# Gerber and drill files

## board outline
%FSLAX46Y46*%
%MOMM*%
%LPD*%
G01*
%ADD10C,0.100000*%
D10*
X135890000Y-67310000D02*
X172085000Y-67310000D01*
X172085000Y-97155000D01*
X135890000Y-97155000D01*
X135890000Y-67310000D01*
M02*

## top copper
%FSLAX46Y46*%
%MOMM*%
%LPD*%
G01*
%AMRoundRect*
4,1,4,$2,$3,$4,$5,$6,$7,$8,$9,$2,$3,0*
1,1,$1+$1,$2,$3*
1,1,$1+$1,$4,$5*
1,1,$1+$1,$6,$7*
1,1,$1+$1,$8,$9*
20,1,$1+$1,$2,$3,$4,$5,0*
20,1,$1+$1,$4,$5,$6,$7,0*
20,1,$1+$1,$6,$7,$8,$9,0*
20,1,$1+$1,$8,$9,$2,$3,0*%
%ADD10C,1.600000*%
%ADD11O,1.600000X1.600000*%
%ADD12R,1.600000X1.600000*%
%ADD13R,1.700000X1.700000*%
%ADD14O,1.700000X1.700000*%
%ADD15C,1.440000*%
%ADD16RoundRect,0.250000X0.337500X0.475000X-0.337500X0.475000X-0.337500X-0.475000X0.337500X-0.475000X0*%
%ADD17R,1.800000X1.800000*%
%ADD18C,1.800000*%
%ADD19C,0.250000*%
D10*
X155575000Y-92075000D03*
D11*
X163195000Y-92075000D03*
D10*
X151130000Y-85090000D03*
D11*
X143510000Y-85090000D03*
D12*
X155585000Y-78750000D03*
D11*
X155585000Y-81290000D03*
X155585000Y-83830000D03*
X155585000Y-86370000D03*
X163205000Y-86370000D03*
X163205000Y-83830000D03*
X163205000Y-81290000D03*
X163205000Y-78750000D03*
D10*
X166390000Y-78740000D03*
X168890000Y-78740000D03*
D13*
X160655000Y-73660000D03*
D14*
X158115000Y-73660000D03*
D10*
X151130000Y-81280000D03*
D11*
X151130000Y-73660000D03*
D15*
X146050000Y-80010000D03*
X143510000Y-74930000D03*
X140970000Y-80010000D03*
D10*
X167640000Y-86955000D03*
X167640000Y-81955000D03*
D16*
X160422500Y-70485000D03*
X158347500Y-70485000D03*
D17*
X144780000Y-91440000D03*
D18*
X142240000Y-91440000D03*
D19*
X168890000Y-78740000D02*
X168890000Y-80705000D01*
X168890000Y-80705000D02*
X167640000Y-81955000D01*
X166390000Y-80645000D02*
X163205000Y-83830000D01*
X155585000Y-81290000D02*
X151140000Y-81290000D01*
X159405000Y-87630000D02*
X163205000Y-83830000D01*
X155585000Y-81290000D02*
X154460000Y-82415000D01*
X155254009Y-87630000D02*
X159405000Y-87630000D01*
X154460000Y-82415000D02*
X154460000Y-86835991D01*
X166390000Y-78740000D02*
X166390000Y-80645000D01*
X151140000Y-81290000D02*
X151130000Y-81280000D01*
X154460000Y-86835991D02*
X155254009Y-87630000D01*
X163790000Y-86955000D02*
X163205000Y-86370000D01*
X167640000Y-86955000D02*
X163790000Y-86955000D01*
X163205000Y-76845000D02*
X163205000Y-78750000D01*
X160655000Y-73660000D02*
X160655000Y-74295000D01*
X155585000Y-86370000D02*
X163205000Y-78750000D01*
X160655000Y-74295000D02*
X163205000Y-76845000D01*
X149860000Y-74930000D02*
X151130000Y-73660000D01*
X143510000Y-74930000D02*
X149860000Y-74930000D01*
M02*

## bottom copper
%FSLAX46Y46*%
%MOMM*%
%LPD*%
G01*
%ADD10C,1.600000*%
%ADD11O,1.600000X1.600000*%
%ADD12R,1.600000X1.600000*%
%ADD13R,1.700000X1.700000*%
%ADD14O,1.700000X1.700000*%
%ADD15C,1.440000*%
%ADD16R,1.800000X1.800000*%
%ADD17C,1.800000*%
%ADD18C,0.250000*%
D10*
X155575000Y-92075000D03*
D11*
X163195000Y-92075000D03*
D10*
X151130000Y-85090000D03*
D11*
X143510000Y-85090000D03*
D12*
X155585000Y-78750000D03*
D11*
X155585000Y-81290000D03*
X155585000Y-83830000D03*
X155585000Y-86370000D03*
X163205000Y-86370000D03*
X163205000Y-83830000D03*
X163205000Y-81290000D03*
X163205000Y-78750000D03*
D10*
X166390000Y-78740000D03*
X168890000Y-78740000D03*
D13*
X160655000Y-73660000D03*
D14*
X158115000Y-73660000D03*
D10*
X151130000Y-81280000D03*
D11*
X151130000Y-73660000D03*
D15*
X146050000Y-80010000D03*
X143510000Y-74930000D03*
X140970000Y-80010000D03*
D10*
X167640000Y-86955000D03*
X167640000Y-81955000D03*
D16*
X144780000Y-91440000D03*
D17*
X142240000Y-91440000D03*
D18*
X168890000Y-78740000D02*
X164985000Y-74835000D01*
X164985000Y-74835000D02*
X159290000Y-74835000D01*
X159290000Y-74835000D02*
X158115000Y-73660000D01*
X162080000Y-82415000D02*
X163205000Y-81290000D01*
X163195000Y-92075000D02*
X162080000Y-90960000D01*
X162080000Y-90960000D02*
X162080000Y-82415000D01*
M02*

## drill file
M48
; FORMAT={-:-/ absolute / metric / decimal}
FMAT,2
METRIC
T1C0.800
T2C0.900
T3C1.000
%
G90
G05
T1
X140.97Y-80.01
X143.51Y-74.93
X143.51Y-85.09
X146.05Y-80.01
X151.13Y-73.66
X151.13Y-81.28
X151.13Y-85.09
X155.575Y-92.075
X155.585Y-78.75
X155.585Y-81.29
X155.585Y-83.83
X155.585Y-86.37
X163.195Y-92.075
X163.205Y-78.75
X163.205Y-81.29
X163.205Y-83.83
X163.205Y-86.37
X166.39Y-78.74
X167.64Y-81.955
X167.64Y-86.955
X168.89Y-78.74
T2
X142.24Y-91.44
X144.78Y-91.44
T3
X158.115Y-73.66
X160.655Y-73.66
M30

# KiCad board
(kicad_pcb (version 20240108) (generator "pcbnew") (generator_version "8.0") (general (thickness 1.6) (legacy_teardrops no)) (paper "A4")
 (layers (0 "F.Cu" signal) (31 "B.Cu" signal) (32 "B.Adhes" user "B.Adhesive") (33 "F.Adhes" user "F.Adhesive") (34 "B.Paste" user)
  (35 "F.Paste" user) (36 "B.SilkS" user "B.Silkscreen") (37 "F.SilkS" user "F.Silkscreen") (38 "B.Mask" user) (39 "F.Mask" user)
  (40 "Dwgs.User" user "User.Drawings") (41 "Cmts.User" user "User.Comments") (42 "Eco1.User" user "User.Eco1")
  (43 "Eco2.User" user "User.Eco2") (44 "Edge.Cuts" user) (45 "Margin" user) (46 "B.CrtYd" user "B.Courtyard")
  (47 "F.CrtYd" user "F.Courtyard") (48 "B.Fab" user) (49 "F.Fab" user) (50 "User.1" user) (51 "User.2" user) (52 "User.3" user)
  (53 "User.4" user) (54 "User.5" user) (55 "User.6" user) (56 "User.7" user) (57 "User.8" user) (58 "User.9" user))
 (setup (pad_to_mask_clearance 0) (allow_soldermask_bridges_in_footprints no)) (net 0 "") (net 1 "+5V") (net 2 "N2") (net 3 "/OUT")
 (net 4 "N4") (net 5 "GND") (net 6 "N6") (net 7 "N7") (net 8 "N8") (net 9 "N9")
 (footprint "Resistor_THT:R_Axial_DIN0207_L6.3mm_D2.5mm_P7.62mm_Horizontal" (layer "F.Cu") (at 155.575 92.075)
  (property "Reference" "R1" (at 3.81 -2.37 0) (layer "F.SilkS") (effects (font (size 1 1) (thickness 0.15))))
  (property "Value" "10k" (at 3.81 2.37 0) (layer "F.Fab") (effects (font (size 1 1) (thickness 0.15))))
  (pad "1" thru_hole circle (at 0 0) (size 1.6 1.6) (drill 0.8) (layers "*.Cu" "*.Mask") (remove_unused_layers no) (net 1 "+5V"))
  (pad "2" thru_hole oval (at 7.62 0) (size 1.6 1.6) (drill 0.8) (layers "*.Cu" "*.Mask") (remove_unused_layers no) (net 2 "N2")))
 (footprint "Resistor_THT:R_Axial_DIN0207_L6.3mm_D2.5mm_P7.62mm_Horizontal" (layer "F.Cu") (at 151.13 85.09 180)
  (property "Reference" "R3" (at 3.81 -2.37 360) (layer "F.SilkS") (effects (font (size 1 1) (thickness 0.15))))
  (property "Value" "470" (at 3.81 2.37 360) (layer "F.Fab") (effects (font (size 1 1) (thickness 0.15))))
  (pad "1" thru_hole circle (at 0 0 180) (size 1.6 1.6) (drill 0.8) (layers "*.Cu" "*.Mask") (remove_unused_layers no) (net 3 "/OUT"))
  (pad "2" thru_hole oval (at 7.62 0 180) (size 1.6 1.6) (drill 0.8) (layers "*.Cu" "*.Mask") (remove_unused_layers no) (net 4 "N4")))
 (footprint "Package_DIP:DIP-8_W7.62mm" (layer "F.Cu") (at 155.585 78.75)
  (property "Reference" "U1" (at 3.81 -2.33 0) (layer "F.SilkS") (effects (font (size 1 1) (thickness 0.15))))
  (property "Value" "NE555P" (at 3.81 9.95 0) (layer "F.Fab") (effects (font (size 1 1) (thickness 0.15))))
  (pad "1" thru_hole rect (at 0 0) (size 1.6 1.6) (drill 0.8) (layers "*.Cu" "*.Mask") (remove_unused_layers no) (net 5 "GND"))
  (pad "2" thru_hole oval (at 0 2.54) (size 1.6 1.6) (drill 0.8) (layers "*.Cu" "*.Mask") (remove_unused_layers no) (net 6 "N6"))
  (pad "3" thru_hole oval (at 0 5.08) (size 1.6 1.6) (drill 0.8) (layers "*.Cu" "*.Mask") (remove_unused_layers no) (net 3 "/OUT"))
  (pad "4" thru_hole oval (at 0 7.62) (size 1.6 1.6) (drill 0.8) (layers "*.Cu" "*.Mask") (remove_unused_layers no) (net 1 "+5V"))
  (pad "5" thru_hole oval (at 7.62 7.62) (size 1.6 1.6) (drill 0.8) (layers "*.Cu" "*.Mask") (remove_unused_layers no) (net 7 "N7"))
  (pad "6" thru_hole oval (at 7.62 5.08) (size 1.6 1.6) (drill 0.8) (layers "*.Cu" "*.Mask") (remove_unused_layers no) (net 6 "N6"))
  (pad "7" thru_hole oval (at 7.62 2.54) (size 1.6 1.6) (drill 0.8) (layers "*.Cu" "*.Mask") (remove_unused_layers no) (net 2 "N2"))
  (pad "8" thru_hole oval (at 7.62 0) (size 1.6 1.6) (drill 0.8) (layers "*.Cu" "*.Mask") (remove_unused_layers no) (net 1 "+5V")))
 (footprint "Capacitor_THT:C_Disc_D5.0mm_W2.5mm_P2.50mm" (layer "F.Cu") (at 166.39 78.74)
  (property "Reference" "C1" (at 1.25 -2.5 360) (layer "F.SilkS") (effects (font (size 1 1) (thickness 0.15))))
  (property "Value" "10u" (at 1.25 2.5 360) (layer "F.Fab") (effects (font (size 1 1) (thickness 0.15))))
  (pad "1" thru_hole circle (at 0 0) (size 1.6 1.6) (drill 0.8) (layers "*.Cu" "*.Mask") (remove_unused_layers no) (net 6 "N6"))
  (pad "2" thru_hole circle (at 2.5 0) (size 1.6 1.6) (drill 0.8) (layers "*.Cu" "*.Mask") (remove_unused_layers no) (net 5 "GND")))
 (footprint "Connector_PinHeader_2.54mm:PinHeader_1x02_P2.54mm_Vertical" (layer "F.Cu") (at 160.655 73.66 -90)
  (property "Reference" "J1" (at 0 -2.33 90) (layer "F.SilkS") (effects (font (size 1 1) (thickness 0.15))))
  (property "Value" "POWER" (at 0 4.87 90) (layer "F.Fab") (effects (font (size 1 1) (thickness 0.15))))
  (pad "1" thru_hole rect (at 0 0 270) (size 1.7 1.7) (drill 1) (layers "*.Cu" "*.Mask") (remove_unused_layers no) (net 1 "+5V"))
  (pad "2" thru_hole oval (at 0 2.54 270) (size 1.7 1.7) (drill 1) (layers "*.Cu" "*.Mask") (remove_unused_layers no) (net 5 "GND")))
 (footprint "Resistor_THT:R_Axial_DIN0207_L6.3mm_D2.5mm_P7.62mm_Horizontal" (layer "F.Cu") (at 151.13 81.28 90)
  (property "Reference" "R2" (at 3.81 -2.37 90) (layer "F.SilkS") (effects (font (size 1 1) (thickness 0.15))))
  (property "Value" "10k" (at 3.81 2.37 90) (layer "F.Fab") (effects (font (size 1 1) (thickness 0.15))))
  (pad "1" thru_hole circle (at 0 0 90) (size 1.6 1.6) (drill 0.8) (layers "*.Cu" "*.Mask") (remove_unused_layers no) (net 6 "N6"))
  (pad "2" thru_hole oval (at 7.62 0 90) (size 1.6 1.6) (drill 0.8) (layers "*.Cu" "*.Mask") (remove_unused_layers no) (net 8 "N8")))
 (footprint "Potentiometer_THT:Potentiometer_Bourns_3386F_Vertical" (layer "F.Cu") (at 146.05 80.01 90)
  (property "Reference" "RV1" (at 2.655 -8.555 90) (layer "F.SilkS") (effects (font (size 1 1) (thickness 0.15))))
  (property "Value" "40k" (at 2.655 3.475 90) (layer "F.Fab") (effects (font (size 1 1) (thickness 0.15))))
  (pad "1" thru_hole circle (at 0 0 90) (size 1.44 1.44) (drill 0.8) (layers "*.Cu" "*.Mask") (remove_unused_layers no) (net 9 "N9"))
  (pad "2" thru_hole circle (at 5.08 -2.54 90) (size 1.44 1.44) (drill 0.8) (layers "*.Cu" "*.Mask") (remove_unused_layers no) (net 8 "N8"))
  (pad "3" thru_hole circle (at 0 -5.08 90) (size 1.44 1.44) (drill 0.8) (layers "*.Cu" "*.Mask") (remove_unused_layers no) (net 2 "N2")))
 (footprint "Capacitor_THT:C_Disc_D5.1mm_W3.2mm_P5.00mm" (layer "F.Cu") (at 167.64 86.955 90)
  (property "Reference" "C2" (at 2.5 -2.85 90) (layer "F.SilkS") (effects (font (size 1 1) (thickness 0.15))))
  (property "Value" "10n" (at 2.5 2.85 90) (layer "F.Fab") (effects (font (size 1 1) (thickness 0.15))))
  (pad "1" thru_hole circle (at 0 0 90) (size 1.6 1.6) (drill 0.8) (layers "*.Cu" "*.Mask") (remove_unused_layers no) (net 7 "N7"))
  (pad "2" thru_hole circle (at 5 0 90) (size 1.6 1.6) (drill 0.8) (layers "*.Cu" "*.Mask") (remove_unused_layers no) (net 5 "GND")))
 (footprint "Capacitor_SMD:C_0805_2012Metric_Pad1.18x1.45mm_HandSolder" (layer "F.Cu") (at 159.385 70.485 180)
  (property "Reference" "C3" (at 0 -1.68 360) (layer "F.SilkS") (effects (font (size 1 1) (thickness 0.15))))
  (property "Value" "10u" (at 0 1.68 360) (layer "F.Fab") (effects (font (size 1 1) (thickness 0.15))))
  (pad "1" smd roundrect (at -1.0375 0 180) (size 1.175 1.45) (layers "F.Cu" "F.Paste" "F.Mask") (roundrect_rratio 0.212766) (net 1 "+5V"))
  (pad "2" smd roundrect (at 1.0375 0 180) (size 1.175 1.45) (layers "F.Cu" "F.Paste" "F.Mask") (roundrect_rratio 0.212766) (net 5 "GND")))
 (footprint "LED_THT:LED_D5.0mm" (layer "F.Cu") (at 144.78 91.44 180)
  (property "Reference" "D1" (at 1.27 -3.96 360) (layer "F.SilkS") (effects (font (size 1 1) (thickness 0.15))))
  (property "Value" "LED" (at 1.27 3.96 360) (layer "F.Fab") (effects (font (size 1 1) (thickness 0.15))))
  (pad "1" thru_hole rect (at 0 0 180) (size 1.8 1.8) (drill 0.9) (layers "*.Cu" "*.Mask") (remove_unused_layers no) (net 5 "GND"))
  (pad "2" thru_hole circle (at 2.54 0 180) (size 1.8 1.8) (drill 0.9) (layers "*.Cu" "*.Mask") (remove_unused_layers no) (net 4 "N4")))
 (gr_rect (start 135.89 67.31) (end 172.085 97.155) (stroke (width 0.1) (type default)) (fill none) (layer "Edge.Cuts"))
 (segment (start 168.89 78.74) (end 168.89 80.705) (width 0.25) (layer "F.Cu") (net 5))
 (segment (start 168.89 80.705) (end 167.64 81.955) (width 0.25) (layer "F.Cu") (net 5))
 (segment (start 168.89 78.74) (end 164.985 74.835) (width 0.25) (layer "B.Cu") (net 5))
 (segment (start 164.985 74.835) (end 159.29 74.835) (width 0.25) (layer "B.Cu") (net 5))
 (segment (start 159.29 74.835) (end 158.115 73.66) (width 0.25) (layer "B.Cu") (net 5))
 (segment (start 166.39 80.645) (end 163.205 83.83) (width 0.25) (layer "F.Cu") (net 6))
 (segment (start 155.585 81.29) (end 151.14 81.29) (width 0.25) (layer "F.Cu") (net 6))
 (segment (start 159.405 87.63) (end 163.205 83.83) (width 0.25) (layer "F.Cu") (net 6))
 (segment (start 155.585 81.29) (end 154.46 82.415) (width 0.25) (layer "F.Cu") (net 6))
 (segment (start 155.254009 87.63) (end 159.405 87.63) (width 0.25) (layer "F.Cu") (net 6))
 (segment (start 154.46 82.415) (end 154.46 86.835991) (width 0.25) (layer "F.Cu") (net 6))
 (segment (start 166.39 78.74) (end 166.39 80.645) (width 0.25) (layer "F.Cu") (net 6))
 (segment (start 151.14 81.29) (end 151.13 81.28) (width 0.25) (layer "F.Cu") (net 6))
 (segment (start 154.46 86.835991) (end 155.254009 87.63) (width 0.25) (layer "F.Cu") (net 6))
 (segment (start 163.79 86.955) (end 163.205 86.37) (width 0.25) (layer "F.Cu") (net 7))
 (segment (start 167.64 86.955) (end 163.79 86.955) (width 0.25) (layer "F.Cu") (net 7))
 (segment (start 163.205 76.845) (end 163.205 78.75) (width 0.25) (layer "F.Cu") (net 1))
 (segment (start 160.655 73.66) (end 160.655 74.295) (width 0.25) (layer "F.Cu") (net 1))
 (segment (start 155.585 86.37) (end 163.205 78.75) (width 0.25) (layer "F.Cu") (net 1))
 (segment (start 160.655 74.295) (end 163.205 76.845) (width 0.25) (layer "F.Cu") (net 1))
 (segment (start 162.08 82.415) (end 163.205 81.29) (width 0.25) (layer "B.Cu") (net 2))
 (segment (start 163.195 92.075) (end 162.08 90.96) (width 0.25) (layer "B.Cu") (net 2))
 (segment (start 162.08 90.96) (end 162.08 82.415) (width 0.25) (layer "B.Cu") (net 2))
 (segment (start 149.86 74.93) (end 151.13 73.66) (width 0.25) (layer "F.Cu") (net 8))
 (segment (start 143.51 74.93) (end 149.86 74.93) (width 0.25) (layer "F.Cu") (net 8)))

